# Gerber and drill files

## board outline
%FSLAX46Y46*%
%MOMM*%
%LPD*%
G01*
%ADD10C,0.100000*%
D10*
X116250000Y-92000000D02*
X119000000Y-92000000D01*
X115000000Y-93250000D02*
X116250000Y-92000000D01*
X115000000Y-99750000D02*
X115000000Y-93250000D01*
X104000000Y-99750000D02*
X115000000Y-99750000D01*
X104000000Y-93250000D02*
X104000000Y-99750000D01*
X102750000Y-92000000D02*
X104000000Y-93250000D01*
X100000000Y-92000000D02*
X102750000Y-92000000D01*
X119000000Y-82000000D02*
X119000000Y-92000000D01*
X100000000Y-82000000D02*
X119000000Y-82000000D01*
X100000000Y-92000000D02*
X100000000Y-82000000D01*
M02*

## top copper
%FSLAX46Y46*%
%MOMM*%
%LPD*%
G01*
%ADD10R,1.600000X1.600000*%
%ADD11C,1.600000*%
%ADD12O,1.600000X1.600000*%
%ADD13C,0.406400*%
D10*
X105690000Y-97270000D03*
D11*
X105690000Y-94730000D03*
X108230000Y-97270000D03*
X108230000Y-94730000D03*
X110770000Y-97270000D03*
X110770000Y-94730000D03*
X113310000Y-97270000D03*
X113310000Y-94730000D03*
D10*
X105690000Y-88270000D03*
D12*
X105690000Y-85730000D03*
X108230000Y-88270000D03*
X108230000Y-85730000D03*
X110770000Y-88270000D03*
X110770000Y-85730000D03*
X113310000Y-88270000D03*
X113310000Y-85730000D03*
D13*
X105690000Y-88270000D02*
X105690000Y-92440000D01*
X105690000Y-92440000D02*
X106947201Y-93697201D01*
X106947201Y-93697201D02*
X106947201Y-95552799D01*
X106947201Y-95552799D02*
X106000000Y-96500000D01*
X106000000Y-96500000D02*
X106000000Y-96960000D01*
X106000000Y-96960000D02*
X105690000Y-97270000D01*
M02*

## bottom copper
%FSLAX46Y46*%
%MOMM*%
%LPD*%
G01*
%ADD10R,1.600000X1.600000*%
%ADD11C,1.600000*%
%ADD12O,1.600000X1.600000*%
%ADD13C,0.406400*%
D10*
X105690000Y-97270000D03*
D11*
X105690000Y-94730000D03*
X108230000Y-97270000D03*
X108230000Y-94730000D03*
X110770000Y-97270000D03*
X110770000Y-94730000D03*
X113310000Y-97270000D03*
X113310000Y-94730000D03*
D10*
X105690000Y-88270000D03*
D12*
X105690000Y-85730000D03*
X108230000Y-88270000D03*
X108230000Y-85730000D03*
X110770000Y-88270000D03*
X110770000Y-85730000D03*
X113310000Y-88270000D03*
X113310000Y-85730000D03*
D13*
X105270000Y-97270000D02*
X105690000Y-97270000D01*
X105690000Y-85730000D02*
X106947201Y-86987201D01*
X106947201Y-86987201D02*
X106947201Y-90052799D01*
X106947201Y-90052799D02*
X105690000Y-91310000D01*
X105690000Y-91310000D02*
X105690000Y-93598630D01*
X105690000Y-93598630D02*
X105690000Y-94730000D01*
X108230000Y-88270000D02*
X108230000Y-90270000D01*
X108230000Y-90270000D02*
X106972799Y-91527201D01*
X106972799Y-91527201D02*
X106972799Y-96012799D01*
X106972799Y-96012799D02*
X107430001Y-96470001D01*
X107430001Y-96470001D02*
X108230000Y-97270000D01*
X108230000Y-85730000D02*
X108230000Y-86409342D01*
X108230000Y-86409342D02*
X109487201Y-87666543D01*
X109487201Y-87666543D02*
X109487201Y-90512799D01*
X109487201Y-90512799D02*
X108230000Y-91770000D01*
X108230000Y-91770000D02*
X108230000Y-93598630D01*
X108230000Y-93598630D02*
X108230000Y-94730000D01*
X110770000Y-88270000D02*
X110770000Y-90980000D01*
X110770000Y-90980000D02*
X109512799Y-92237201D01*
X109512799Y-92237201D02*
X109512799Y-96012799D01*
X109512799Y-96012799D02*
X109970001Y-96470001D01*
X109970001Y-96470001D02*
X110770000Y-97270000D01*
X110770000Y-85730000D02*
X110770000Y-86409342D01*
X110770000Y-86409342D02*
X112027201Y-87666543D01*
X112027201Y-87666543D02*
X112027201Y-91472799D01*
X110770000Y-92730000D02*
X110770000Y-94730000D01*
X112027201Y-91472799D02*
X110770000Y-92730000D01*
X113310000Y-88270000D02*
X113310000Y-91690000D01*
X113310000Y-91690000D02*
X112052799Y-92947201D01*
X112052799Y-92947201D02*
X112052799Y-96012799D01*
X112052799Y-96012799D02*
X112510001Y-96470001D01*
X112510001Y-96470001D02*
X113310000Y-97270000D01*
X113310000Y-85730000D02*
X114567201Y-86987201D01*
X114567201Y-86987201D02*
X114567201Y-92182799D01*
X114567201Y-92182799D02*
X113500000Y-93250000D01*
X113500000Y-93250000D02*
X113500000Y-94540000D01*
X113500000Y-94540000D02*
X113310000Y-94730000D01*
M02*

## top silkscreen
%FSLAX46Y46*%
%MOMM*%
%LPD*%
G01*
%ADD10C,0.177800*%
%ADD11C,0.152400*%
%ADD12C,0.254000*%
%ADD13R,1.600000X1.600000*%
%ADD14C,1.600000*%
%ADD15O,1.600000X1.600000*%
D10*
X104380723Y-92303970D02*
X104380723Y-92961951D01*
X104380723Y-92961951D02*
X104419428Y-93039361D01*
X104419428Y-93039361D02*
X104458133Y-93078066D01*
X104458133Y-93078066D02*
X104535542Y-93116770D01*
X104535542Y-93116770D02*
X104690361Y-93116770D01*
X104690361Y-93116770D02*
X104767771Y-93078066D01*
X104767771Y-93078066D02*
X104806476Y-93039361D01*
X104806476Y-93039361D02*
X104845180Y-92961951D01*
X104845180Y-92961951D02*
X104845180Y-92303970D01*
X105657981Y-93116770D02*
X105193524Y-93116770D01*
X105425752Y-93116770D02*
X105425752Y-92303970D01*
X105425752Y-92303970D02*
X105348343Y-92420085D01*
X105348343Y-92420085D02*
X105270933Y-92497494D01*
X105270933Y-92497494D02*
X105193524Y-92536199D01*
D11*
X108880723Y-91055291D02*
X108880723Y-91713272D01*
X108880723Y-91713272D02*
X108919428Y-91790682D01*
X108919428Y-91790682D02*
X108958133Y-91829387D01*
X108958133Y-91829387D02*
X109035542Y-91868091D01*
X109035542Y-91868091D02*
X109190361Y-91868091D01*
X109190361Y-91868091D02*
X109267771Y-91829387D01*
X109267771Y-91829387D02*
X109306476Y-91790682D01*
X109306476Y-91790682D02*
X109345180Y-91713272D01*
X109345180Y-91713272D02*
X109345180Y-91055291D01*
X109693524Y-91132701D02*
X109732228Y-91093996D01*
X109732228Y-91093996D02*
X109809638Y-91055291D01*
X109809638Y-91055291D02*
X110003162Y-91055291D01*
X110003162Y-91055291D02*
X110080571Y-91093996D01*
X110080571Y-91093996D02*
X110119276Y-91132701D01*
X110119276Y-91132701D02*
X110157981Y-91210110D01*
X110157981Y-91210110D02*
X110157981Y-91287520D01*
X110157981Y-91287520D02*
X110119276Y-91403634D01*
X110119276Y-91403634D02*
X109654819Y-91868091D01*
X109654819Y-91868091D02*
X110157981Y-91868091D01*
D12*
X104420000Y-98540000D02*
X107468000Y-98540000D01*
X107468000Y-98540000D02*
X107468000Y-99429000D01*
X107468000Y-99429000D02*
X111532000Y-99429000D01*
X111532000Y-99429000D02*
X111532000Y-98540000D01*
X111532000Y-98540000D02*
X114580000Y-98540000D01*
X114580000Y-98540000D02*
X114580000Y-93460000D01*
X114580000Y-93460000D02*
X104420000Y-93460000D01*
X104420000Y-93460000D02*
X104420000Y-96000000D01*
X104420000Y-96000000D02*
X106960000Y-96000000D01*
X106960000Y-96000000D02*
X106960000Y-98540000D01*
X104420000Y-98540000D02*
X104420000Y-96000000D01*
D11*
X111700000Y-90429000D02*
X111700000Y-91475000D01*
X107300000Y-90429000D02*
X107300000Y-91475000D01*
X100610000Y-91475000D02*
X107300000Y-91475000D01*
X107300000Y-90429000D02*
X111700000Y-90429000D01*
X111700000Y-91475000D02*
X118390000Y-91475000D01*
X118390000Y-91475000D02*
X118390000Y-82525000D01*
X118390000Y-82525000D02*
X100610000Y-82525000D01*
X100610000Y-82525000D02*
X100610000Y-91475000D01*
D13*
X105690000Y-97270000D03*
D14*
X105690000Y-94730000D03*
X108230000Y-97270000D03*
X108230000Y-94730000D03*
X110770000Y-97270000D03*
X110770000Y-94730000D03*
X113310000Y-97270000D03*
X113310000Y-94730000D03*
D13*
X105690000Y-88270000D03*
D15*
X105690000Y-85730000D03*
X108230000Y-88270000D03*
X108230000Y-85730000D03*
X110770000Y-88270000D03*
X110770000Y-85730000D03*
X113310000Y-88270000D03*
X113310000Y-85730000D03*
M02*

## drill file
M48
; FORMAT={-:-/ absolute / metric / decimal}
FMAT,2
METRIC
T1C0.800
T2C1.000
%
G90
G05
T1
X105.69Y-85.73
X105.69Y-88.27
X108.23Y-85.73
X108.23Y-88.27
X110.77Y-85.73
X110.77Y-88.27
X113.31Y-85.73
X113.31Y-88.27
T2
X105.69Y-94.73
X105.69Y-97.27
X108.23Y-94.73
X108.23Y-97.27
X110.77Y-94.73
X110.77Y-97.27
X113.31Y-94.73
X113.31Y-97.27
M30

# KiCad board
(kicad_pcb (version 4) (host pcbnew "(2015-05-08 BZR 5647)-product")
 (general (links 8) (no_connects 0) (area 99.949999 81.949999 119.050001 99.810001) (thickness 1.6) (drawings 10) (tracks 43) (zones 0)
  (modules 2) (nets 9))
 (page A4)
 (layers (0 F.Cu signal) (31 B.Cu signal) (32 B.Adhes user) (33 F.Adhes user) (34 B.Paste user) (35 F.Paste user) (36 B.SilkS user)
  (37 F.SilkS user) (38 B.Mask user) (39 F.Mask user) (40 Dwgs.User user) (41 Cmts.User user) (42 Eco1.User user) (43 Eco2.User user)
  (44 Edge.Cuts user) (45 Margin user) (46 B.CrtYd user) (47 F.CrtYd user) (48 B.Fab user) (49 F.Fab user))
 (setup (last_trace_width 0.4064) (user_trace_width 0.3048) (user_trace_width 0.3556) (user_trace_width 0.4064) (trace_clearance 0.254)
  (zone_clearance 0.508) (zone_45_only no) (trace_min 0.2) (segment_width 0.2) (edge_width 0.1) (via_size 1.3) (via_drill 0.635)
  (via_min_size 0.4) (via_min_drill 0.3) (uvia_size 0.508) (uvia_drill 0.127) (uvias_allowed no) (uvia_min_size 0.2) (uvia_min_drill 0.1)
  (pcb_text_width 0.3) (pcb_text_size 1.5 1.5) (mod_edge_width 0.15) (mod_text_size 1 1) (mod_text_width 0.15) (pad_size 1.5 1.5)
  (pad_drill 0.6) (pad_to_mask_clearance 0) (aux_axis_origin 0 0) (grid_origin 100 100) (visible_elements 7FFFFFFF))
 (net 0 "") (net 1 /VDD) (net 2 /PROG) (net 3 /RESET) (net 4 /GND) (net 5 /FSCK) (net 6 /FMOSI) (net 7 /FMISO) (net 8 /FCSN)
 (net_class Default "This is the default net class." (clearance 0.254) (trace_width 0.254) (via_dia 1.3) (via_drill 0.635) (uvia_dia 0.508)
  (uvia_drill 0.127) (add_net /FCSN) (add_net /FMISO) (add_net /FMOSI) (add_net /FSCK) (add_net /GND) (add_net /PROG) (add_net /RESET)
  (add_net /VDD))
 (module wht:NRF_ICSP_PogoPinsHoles (layer F.Cu) (at 109.5 96)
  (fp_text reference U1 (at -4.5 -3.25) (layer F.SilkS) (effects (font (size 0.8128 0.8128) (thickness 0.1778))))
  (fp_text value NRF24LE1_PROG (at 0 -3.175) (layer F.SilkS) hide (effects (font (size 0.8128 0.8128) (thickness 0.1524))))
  (fp_line (start -5.08 2.54) (end -2.032 2.54) (layer F.SilkS) (width 0.254))
  (fp_line (start -2.032 2.54) (end -2.032 3.429) (layer F.SilkS) (width 0.254))
  (fp_line (start -2.032 3.429) (end 2.032 3.429) (layer F.SilkS) (width 0.254))
  (fp_line (start 2.032 3.429) (end 2.032 2.54) (layer F.SilkS) (width 0.254))
  (fp_line (start 2.032 2.54) (end 5.08 2.54) (layer F.SilkS) (width 0.254))
  (fp_line (start 5.08 2.54) (end 5.08 -2.54) (layer F.SilkS) (width 0.254))
  (fp_line (start 5.08 -2.54) (end -5.08 -2.54) (layer F.SilkS) (width 0.254))
  (fp_line (start -5.08 -2.54) (end -5.08 0) (layer F.SilkS) (width 0.254))
  (fp_line (start -5.08 0) (end -2.54 0) (layer F.SilkS) (width 0.254))
  (fp_line (start -2.54 0) (end -2.54 2.54) (layer F.SilkS) (width 0.254))
  (fp_line (start -5.08 2.54) (end -5.08 0) (layer F.SilkS) (width 0.254))
  (pad 1 thru_hole rect (at -3.81 1.27) (size 1.6 1.6) (drill 1) (layers *.Cu *.Mask F.SilkS) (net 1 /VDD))
  (pad 2 thru_hole circle (at -3.81 -1.27) (size 1.6 1.6) (drill 1) (layers *.Cu *.Mask F.SilkS) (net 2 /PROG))
  (pad 3 thru_hole circle (at -1.27 1.27) (size 1.6 1.6) (drill 1) (layers *.Cu *.Mask F.SilkS) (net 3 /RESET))
  (pad 4 thru_hole circle (at -1.27 -1.27) (size 1.6 1.6) (drill 1) (layers *.Cu *.Mask F.SilkS) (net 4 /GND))
  (pad 5 thru_hole circle (at 1.27 1.27) (size 1.6 1.6) (drill 1) (layers *.Cu *.Mask F.SilkS) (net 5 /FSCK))
  (pad 6 thru_hole circle (at 1.27 -1.27) (size 1.6 1.6) (drill 1) (layers *.Cu *.Mask F.SilkS) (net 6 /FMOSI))
  (pad 7 thru_hole circle (at 3.81 1.27) (size 1.6 1.6) (drill 1) (layers *.Cu *.Mask F.SilkS) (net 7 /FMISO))
  (pad 8 thru_hole circle (at 3.81 -1.27) (size 1.6 1.6) (drill 1) (layers *.Cu *.Mask F.SilkS) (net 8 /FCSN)))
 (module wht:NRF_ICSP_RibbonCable (layer F.Cu) (at 109.5 87)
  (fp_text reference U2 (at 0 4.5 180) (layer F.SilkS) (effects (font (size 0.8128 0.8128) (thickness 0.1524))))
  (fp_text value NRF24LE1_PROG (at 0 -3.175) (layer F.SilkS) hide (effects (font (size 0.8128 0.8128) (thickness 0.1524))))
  (fp_line (start 2.2 3.429) (end 2.2 4.475) (layer F.SilkS) (width 0.1524))
  (fp_line (start -2.2 3.429) (end -2.2 4.475) (layer F.SilkS) (width 0.1524))
  (fp_line (start -8.89 4.475) (end -2.2 4.475) (layer F.SilkS) (width 0.1524))
  (fp_line (start -2.2 3.429) (end 2.2 3.429) (layer F.SilkS) (width 0.1524))
  (fp_line (start 2.2 4.475) (end 8.89 4.475) (layer F.SilkS) (width 0.1524))
  (fp_line (start 8.89 4.475) (end 8.89 -4.475) (layer F.SilkS) (width 0.1524))
  (fp_line (start 8.89 -4.475) (end -8.89 -4.475) (layer F.SilkS) (width 0.1524))
  (fp_line (start -8.89 -4.475) (end -8.89 4.475) (layer F.SilkS) (width 0.1524))
  (pad 1 thru_hole rect (at -3.81 1.27) (size 1.6 1.6) (drill 0.8) (layers *.Cu *.Mask F.SilkS) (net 1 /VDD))
  (pad 2 thru_hole oval (at -3.81 -1.27) (size 1.6 1.6) (drill 0.8) (layers *.Cu *.Mask F.SilkS) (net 2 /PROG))
  (pad 3 thru_hole oval (at -1.27 1.27) (size 1.6 1.6) (drill 0.8) (layers *.Cu *.Mask F.SilkS) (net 3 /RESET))
  (pad 4 thru_hole oval (at -1.27 -1.27) (size 1.6 1.6) (drill 0.8) (layers *.Cu *.Mask F.SilkS) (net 4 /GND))
  (pad 5 thru_hole oval (at 1.27 1.27) (size 1.6 1.6) (drill 0.8) (layers *.Cu *.Mask F.SilkS) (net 5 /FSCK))
  (pad 6 thru_hole oval (at 1.27 -1.27) (size 1.6 1.6) (drill 0.8) (layers *.Cu *.Mask F.SilkS) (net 6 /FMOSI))
  (pad 7 thru_hole oval (at 3.81 1.27) (size 1.6 1.6) (drill 0.8) (layers *.Cu *.Mask F.SilkS) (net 7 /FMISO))
  (pad 8 thru_hole oval (at 3.81 -1.27) (size 1.6 1.6) (drill 0.8) (layers *.Cu *.Mask F.SilkS) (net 8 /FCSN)))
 (gr_line (start 116.25 92) (end 119 92) (angle 90) (layer Edge.Cuts) (width 0.1))
 (gr_line (start 115 93.25) (end 116.25 92) (angle 90) (layer Edge.Cuts) (width 0.1))
 (gr_line (start 115 99.75) (end 115 93.25) (angle 90) (layer Edge.Cuts) (width 0.1))
 (gr_line (start 104 99.75) (end 115 99.75) (angle 90) (layer Edge.Cuts) (width 0.1))
 (gr_line (start 104 93.25) (end 104 99.75) (angle 90) (layer Edge.Cuts) (width 0.1))
 (gr_line (start 102.75 92) (end 104 93.25) (angle 90) (layer Edge.Cuts) (width 0.1))
 (gr_line (start 100 92) (end 102.75 92) (angle 90) (layer Edge.Cuts) (width 0.1))
 (gr_line (start 119 82) (end 119 92) (angle 90) (layer Edge.Cuts) (width 0.1))
 (gr_line (start 100 82) (end 119 82) (angle 90) (layer Edge.Cuts) (width 0.1))
 (gr_line (start 100 92) (end 100 82) (angle 90) (layer Edge.Cuts) (width 0.1))
 (segment (start 105.69 88.27) (end 105.69 92.44) (width 0.4064) (layer F.Cu) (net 1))
 (segment (start 105.69 92.44) (end 106.947201 93.697201) (width 0.4064) (layer F.Cu) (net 1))
 (segment (start 106.947201 93.697201) (end 106.947201 95.552799) (width 0.4064) (layer F.Cu) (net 1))
 (segment (start 106.947201 95.552799) (end 106 96.5) (width 0.4064) (layer F.Cu) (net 1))
 (segment (start 106 96.5) (end 106 96.96) (width 0.4064) (layer F.Cu) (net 1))
 (segment (start 106 96.96) (end 105.69 97.27) (width 0.4064) (layer F.Cu) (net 1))
 (segment (start 105.27 97.27) (end 105.69 97.27) (width 0.4064) (layer B.Cu) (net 1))
 (segment (start 105.69 85.73) (end 106.947201 86.987201) (width 0.4064) (layer B.Cu) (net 2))
 (segment (start 106.947201 86.987201) (end 106.947201 90.052799) (width 0.4064) (layer B.Cu) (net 2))
 (segment (start 106.947201 90.052799) (end 105.69 91.31) (width 0.4064) (layer B.Cu) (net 2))
 (segment (start 105.69 91.31) (end 105.69 93.59863) (width 0.4064) (layer B.Cu) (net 2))
 (segment (start 105.69 93.59863) (end 105.69 94.73) (width 0.4064) (layer B.Cu) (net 2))
 (segment (start 108.23 88.27) (end 108.23 90.27) (width 0.4064) (layer B.Cu) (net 3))
 (segment (start 108.23 90.27) (end 106.972799 91.527201) (width 0.4064) (layer B.Cu) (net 3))
 (segment (start 106.972799 91.527201) (end 106.972799 96.012799) (width 0.4064) (layer B.Cu) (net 3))
 (segment (start 106.972799 96.012799) (end 107.430001 96.470001) (width 0.4064) (layer B.Cu) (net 3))
 (segment (start 107.430001 96.470001) (end 108.23 97.27) (width 0.4064) (layer B.Cu) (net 3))
 (segment (start 108.23 85.73) (end 108.23 86.409342) (width 0.4064) (layer B.Cu) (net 4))
 (segment (start 108.23 86.409342) (end 109.487201 87.666543) (width 0.4064) (layer B.Cu) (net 4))
 (segment (start 109.487201 87.666543) (end 109.487201 90.512799) (width 0.4064) (layer B.Cu) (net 4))
 (segment (start 109.487201 90.512799) (end 108.23 91.77) (width 0.4064) (layer B.Cu) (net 4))
 (segment (start 108.23 91.77) (end 108.23 93.59863) (width 0.4064) (layer B.Cu) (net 4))
 (segment (start 108.23 93.59863) (end 108.23 94.73) (width 0.4064) (layer B.Cu) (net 4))
 (segment (start 110.77 88.27) (end 110.77 90.98) (width 0.4064) (layer B.Cu) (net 5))
 (segment (start 110.77 90.98) (end 109.512799 92.237201) (width 0.4064) (layer B.Cu) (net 5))
 (segment (start 109.512799 92.237201) (end 109.512799 96.012799) (width 0.4064) (layer B.Cu) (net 5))
 (segment (start 109.512799 96.012799) (end 109.970001 96.470001) (width 0.4064) (layer B.Cu) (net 5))
 (segment (start 109.970001 96.470001) (end 110.77 97.27) (width 0.4064) (layer B.Cu) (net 5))
 (segment (start 110.77 85.73) (end 110.77 86.409342) (width 0.4064) (layer B.Cu) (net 6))
 (segment (start 110.77 86.409342) (end 112.027201 87.666543) (width 0.4064) (layer B.Cu) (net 6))
 (segment (start 112.027201 87.666543) (end 112.027201 91.472799) (width 0.4064) (layer B.Cu) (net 6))
 (segment (start 110.77 92.73) (end 110.77 94.73) (width 0.4064) (layer B.Cu) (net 6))
 (segment (start 112.027201 91.472799) (end 110.77 92.73) (width 0.4064) (layer B.Cu) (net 6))
 (segment (start 113.31 88.27) (end 113.31 91.69) (width 0.4064) (layer B.Cu) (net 7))
 (segment (start 113.31 91.69) (end 112.052799 92.947201) (width 0.4064) (layer B.Cu) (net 7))
 (segment (start 112.052799 92.947201) (end 112.052799 96.012799) (width 0.4064) (layer B.Cu) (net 7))
 (segment (start 112.052799 96.012799) (end 112.510001 96.470001) (width 0.4064) (layer B.Cu) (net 7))
 (segment (start 112.510001 96.470001) (end 113.31 97.27) (width 0.4064) (layer B.Cu) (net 7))
 (segment (start 113.31 85.73) (end 114.567201 86.987201) (width 0.4064) (layer B.Cu) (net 8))
 (segment (start 114.567201 86.987201) (end 114.567201 92.182799) (width 0.4064) (layer B.Cu) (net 8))
 (segment (start 114.567201 92.182799) (end 113.5 93.25) (width 0.4064) (layer B.Cu) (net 8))
 (segment (start 113.5 93.25) (end 113.5 94.54) (width 0.4064) (layer B.Cu) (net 8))
 (segment (start 113.5 94.54) (end 113.31 94.73) (width 0.4064) (layer B.Cu) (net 8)))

